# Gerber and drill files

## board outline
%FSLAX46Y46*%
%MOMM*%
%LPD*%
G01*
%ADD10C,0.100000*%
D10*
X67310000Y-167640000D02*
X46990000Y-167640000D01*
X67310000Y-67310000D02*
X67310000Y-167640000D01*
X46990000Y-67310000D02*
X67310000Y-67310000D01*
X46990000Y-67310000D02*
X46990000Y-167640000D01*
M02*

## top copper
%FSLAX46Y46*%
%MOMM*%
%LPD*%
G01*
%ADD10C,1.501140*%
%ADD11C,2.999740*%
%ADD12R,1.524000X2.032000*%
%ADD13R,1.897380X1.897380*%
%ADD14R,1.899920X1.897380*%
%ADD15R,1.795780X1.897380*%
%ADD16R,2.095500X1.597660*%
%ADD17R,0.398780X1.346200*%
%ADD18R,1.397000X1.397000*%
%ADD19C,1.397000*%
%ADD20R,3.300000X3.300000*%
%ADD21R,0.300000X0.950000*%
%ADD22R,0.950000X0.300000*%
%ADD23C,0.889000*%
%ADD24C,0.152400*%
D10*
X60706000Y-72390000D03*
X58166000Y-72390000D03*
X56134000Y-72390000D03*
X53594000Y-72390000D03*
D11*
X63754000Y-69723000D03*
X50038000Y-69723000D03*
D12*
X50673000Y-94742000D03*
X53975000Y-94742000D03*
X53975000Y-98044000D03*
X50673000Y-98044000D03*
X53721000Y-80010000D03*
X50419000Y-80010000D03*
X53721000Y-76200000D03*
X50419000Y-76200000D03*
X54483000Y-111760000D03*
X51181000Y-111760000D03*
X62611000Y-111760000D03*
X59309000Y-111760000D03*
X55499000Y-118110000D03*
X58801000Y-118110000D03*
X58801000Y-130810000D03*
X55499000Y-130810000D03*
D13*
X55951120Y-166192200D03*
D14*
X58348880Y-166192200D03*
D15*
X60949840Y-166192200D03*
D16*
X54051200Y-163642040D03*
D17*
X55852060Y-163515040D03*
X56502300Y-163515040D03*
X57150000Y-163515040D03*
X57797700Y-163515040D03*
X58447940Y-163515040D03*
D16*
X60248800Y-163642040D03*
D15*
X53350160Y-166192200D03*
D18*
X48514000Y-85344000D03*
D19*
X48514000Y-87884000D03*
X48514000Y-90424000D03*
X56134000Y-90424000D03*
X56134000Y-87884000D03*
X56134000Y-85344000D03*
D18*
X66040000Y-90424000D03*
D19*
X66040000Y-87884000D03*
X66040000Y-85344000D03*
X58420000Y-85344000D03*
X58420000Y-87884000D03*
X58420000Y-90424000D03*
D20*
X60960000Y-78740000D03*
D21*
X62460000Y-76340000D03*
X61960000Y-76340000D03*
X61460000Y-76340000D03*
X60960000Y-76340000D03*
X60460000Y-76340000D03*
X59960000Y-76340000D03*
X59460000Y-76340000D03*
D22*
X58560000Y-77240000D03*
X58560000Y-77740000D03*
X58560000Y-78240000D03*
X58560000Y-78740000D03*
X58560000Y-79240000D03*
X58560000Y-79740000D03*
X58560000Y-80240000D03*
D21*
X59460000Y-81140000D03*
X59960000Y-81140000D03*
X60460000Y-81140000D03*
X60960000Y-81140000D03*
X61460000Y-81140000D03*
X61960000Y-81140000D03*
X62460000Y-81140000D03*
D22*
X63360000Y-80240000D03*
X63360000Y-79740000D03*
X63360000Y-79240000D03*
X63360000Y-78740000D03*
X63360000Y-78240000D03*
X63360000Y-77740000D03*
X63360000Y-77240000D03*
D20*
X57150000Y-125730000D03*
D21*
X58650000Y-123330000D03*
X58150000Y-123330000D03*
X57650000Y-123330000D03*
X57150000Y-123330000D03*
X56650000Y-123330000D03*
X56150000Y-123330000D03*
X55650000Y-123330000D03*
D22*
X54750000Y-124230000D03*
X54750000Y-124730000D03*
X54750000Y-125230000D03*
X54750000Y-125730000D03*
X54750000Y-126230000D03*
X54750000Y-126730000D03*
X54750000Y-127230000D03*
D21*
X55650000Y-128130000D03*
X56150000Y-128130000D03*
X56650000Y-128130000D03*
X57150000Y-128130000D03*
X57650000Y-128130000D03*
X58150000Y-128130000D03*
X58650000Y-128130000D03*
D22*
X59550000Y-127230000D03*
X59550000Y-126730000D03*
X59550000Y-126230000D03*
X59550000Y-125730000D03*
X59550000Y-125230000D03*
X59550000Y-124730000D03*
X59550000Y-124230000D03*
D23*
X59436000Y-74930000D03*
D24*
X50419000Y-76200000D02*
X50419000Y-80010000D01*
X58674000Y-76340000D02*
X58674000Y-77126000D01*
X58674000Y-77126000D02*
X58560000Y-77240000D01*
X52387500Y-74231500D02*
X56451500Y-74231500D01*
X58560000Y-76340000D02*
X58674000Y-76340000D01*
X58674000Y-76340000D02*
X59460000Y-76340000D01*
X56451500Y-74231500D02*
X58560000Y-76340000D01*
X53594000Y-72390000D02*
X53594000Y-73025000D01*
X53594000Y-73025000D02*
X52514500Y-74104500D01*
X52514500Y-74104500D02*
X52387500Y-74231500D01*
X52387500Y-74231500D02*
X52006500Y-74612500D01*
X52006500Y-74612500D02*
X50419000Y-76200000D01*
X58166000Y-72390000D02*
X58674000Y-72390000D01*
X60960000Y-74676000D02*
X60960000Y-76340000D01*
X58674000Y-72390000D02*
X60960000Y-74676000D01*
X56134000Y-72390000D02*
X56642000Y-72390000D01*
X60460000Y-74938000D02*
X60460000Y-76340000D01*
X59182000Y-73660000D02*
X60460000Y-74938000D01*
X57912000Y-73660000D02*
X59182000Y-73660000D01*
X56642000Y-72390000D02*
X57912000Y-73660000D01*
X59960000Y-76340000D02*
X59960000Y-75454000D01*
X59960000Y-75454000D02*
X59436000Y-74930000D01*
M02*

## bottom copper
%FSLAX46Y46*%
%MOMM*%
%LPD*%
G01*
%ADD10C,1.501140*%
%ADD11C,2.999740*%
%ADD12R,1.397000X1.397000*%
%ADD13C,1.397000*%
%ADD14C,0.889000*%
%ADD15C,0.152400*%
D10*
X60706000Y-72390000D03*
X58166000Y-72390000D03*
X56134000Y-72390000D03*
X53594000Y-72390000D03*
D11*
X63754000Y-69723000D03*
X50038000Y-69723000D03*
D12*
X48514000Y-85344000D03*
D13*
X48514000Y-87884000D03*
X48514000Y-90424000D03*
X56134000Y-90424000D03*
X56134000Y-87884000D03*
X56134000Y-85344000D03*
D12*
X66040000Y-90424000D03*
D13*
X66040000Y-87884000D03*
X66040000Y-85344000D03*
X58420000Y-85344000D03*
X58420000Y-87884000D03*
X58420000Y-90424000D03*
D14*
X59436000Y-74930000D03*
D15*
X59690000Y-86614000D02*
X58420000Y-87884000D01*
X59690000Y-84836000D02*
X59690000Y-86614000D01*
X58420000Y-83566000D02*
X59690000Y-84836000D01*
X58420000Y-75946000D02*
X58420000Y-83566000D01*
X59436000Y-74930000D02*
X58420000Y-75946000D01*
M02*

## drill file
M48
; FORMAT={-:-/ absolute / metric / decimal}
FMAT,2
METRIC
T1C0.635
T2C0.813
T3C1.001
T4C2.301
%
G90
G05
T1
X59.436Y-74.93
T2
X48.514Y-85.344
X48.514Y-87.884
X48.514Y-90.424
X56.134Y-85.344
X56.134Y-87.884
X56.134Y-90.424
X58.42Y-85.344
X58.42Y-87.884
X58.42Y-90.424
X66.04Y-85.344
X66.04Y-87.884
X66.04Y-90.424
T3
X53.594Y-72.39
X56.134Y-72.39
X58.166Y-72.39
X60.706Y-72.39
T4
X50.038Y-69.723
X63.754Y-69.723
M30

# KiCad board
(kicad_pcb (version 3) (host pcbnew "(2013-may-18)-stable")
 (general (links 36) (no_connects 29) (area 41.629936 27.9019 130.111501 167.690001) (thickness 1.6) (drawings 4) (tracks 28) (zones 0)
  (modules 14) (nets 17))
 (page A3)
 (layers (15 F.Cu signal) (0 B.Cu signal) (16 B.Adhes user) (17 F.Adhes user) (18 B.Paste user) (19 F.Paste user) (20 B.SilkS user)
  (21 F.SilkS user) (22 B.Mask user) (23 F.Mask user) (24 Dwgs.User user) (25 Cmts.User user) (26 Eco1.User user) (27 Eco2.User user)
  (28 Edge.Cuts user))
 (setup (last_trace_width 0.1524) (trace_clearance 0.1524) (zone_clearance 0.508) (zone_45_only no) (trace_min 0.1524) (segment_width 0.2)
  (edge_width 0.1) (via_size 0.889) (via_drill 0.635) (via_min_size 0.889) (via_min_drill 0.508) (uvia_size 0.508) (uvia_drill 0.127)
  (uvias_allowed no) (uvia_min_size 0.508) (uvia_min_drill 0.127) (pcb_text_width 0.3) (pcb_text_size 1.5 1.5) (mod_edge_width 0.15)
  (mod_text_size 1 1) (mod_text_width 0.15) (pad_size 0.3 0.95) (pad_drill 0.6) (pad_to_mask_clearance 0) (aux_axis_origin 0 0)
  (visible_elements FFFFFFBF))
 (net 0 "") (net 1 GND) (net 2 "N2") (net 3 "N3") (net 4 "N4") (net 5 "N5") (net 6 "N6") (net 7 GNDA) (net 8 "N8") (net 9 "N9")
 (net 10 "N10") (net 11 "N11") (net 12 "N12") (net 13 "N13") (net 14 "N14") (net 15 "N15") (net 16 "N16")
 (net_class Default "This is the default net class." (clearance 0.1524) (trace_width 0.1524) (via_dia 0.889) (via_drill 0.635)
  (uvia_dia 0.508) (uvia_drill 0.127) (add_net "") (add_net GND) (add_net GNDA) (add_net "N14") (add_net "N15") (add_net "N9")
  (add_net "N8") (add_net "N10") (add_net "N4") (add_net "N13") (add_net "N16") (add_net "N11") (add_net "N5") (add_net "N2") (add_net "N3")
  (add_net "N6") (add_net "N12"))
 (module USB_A (layer B.Cu) (at 57.15 72.39 90)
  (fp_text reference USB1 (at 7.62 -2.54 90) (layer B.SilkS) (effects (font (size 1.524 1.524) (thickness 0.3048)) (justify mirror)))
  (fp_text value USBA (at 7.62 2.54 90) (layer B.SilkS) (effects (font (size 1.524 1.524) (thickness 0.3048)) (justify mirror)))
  (pad 4 thru_hole circle (at 0 3.556 90) (size 1.50114 1.50114) (drill 1.00076) (layers *.Cu *.Mask B.SilkS) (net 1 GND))
  (pad 3 thru_hole circle (at 0 1.016 90) (size 1.50114 1.50114) (drill 1.00076) (layers *.Cu *.Mask B.SilkS) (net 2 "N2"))
  (pad 2 thru_hole circle (at 0 -1.016 90) (size 1.50114 1.50114) (drill 1.00076) (layers *.Cu *.Mask B.SilkS) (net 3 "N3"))
  (pad 1 thru_hole circle (at 0 -3.556 90) (size 1.50114 1.50114) (drill 1.00076) (layers *.Cu *.Mask B.SilkS) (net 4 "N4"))
  (pad 5 thru_hole circle (at 2.667 6.604 90) (size 2.99974 2.99974) (drill 2.30124) (layers *.Cu *.Mask B.SilkS))
  (pad 6 thru_hole circle (at 2.667 -7.112 90) (size 2.99974 2.99974) (drill 2.30124) (layers *.Cu *.Mask B.SilkS)))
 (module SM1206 (layer F.Cu) (at 52.324 94.742)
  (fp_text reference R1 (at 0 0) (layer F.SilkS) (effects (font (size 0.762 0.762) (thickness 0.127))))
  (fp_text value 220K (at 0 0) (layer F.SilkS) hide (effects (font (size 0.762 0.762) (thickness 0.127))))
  (pad 1 smd rect (at -1.651 0) (size 1.524 2.032) (layers F.Cu F.Paste F.Mask) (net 1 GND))
  (pad 2 smd rect (at 1.651 0) (size 1.524 2.032) (layers F.Cu F.Paste F.Mask) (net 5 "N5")))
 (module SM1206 (layer F.Cu) (at 52.324 98.044 180)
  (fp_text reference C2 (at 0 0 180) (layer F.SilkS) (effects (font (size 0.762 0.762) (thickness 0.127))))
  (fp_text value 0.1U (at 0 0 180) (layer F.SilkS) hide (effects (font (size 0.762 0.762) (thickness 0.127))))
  (pad 1 smd rect (at -1.651 0 180) (size 1.524 2.032) (layers F.Cu F.Paste F.Mask) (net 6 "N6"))
  (pad 2 smd rect (at 1.651 0 180) (size 1.524 2.032) (layers F.Cu F.Paste F.Mask) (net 1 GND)))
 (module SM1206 (layer F.Cu) (at 52.07 80.01 180)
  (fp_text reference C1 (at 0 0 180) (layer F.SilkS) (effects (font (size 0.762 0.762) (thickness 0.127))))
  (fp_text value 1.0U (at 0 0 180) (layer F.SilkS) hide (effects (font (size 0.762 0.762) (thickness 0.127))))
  (pad 1 smd rect (at -1.651 0 180) (size 1.524 2.032) (layers F.Cu F.Paste F.Mask) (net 1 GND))
  (pad 2 smd rect (at 1.651 0 180) (size 1.524 2.032) (layers F.Cu F.Paste F.Mask) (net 4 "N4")))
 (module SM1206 (layer F.Cu) (at 52.07 76.2 180)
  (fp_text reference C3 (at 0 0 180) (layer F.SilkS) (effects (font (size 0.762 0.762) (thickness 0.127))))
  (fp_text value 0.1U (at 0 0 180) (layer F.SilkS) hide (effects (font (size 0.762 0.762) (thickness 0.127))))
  (pad 1 smd rect (at -1.651 0 180) (size 1.524 2.032) (layers F.Cu F.Paste F.Mask) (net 1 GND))
  (pad 2 smd rect (at 1.651 0 180) (size 1.524 2.032) (layers F.Cu F.Paste F.Mask) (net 4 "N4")))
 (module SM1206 (layer F.Cu) (at 52.832 111.76 180)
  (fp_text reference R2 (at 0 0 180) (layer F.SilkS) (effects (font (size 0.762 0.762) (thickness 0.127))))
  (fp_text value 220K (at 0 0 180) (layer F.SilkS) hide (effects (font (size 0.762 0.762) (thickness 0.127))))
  (pad 1 smd rect (at -1.651 0 180) (size 1.524 2.032) (layers F.Cu F.Paste F.Mask) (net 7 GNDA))
  (pad 2 smd rect (at 1.651 0 180) (size 1.524 2.032) (layers F.Cu F.Paste F.Mask) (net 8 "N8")))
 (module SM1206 (layer F.Cu) (at 60.96 111.76 180)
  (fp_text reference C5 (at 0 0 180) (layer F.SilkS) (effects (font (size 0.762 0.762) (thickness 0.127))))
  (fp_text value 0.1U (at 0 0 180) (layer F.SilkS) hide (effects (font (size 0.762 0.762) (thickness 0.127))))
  (pad 1 smd rect (at -1.651 0 180) (size 1.524 2.032) (layers F.Cu F.Paste F.Mask) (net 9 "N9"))
  (pad 2 smd rect (at 1.651 0 180) (size 1.524 2.032) (layers F.Cu F.Paste F.Mask) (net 7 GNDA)))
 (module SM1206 (layer F.Cu) (at 57.15 118.11)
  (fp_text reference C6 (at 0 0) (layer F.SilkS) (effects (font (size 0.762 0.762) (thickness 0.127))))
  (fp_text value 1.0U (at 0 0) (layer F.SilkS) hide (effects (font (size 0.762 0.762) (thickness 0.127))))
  (pad 1 smd rect (at -1.651 0) (size 1.524 2.032) (layers F.Cu F.Paste F.Mask) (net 7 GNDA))
  (pad 2 smd rect (at 1.651 0) (size 1.524 2.032) (layers F.Cu F.Paste F.Mask) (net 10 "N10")))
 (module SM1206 (layer F.Cu) (at 57.15 130.81 180)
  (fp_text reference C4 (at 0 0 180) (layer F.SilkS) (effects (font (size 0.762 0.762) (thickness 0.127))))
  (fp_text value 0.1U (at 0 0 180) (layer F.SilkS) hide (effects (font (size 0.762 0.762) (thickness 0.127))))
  (pad 1 smd rect (at -1.651 0 180) (size 1.524 2.032) (layers F.Cu F.Paste F.Mask) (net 7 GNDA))
  (pad 2 smd rect (at 1.651 0 180) (size 1.524 2.032) (layers F.Cu F.Paste F.Mask) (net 10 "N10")))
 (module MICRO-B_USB (layer F.Cu) (at 57.15 167.64)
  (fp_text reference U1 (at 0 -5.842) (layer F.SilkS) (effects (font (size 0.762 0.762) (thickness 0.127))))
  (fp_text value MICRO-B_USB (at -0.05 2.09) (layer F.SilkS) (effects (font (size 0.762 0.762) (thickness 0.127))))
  (pad "" smd rect (at -1.19888 -1.4478) (size 1.89738 1.89738) (layers F.Cu F.Paste F.Mask))
  (pad "" smd rect (at 1.19888 -1.4478) (size 1.89992 1.89738) (layers F.Cu F.Paste F.Mask))
  (pad "" smd rect (at 3.79984 -1.4478) (size 1.79578 1.89738) (layers F.Cu F.Paste F.Mask))
  (pad "" smd rect (at -3.0988 -3.99796) (size 2.0955 1.59766) (layers F.Cu F.Paste F.Mask))
  (pad 1 smd rect (at -1.29794 -4.12496) (size 0.39878 1.3462) (layers F.Cu F.Paste F.Mask) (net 10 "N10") (clearance 0.2032))
  (pad 2 smd rect (at -0.6477 -4.12496) (size 0.39878 1.3462) (layers F.Cu F.Paste F.Mask) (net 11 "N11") (clearance 0.2032))
  (pad 3 smd rect (at 0 -4.12496) (size 0.39878 1.3462) (layers F.Cu F.Paste F.Mask) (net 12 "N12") (clearance 0.2032))
  (pad 4 smd rect (at 0.6477 -4.12496) (size 0.39878 1.3462) (layers F.Cu F.Paste F.Mask) (clearance 0.2032))
  (pad 5 smd rect (at 1.29794 -4.12496) (size 0.39878 1.3462) (layers F.Cu F.Paste F.Mask) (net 7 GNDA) (clearance 0.2032))
  (pad "" smd rect (at 3.0988 -3.99796) (size 2.0955 1.59766) (layers F.Cu F.Paste F.Mask))
  (pad "" smd rect (at -3.79984 -1.4478) (size 1.79578 1.89738) (layers F.Cu F.Paste F.Mask)))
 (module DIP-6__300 (layer F.Cu) (at 52.324 87.884 270)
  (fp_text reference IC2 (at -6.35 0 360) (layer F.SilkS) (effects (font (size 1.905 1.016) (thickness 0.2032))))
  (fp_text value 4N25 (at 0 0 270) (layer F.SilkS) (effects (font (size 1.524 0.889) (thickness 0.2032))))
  (pad 1 thru_hole rect (at -2.54 3.81 270) (size 1.397 1.397) (drill 0.8128) (layers *.Cu *.Mask F.SilkS) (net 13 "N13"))
  (pad 2 thru_hole circle (at 0 3.81 270) (size 1.397 1.397) (drill 0.8128) (layers *.Cu *.Mask F.SilkS) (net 1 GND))
  (pad 3 thru_hole circle (at 2.54 3.81 270) (size 1.397 1.397) (drill 0.8128) (layers *.Cu *.Mask F.SilkS))
  (pad 4 thru_hole circle (at 2.54 -3.81 270) (size 1.397 1.397) (drill 0.8128) (layers *.Cu *.Mask F.SilkS) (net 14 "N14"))
  (pad 5 thru_hole circle (at 0 -3.81 270) (size 1.397 1.397) (drill 0.8128) (layers *.Cu *.Mask F.SilkS) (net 9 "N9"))
  (pad 6 thru_hole circle (at -2.54 -3.81 270) (size 1.397 1.397) (drill 0.8128) (layers *.Cu *.Mask F.SilkS) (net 8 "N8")))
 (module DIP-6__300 (layer F.Cu) (at 62.23 87.884 90)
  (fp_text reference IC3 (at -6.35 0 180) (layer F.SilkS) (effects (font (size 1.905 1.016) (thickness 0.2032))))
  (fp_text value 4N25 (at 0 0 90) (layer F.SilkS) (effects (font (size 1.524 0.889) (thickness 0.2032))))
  (pad 1 thru_hole rect (at -2.54 3.81 90) (size 1.397 1.397) (drill 0.8128) (layers *.Cu *.Mask F.SilkS) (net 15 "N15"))
  (pad 2 thru_hole circle (at 0 3.81 90) (size 1.397 1.397) (drill 0.8128) (layers *.Cu *.Mask F.SilkS) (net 7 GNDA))
  (pad 3 thru_hole circle (at 2.54 3.81 90) (size 1.397 1.397) (drill 0.8128) (layers *.Cu *.Mask F.SilkS))
  (pad 4 thru_hole circle (at 2.54 -3.81 90) (size 1.397 1.397) (drill 0.8128) (layers *.Cu *.Mask F.SilkS) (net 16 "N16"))
  (pad 5 thru_hole circle (at 0 -3.81 90) (size 1.397 1.397) (drill 0.8128) (layers *.Cu *.Mask F.SilkS) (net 6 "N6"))
  (pad 6 thru_hole circle (at -2.54 -3.81 90) (size 1.397 1.397) (drill 0.8128) (layers *.Cu *.Mask F.SilkS) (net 5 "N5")))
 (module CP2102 (layer F.Cu) (at 60.96 78.74 270)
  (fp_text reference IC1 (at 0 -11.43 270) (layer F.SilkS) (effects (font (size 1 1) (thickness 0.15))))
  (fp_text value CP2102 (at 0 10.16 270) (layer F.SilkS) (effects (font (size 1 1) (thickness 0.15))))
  (pad 3 smd rect (at 0 0 270) (size 3.3 3.3) (layers F.Cu F.Paste F.Mask) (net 1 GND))
  (pad 1 smd rect (at -2.4 -1.5 270) (size 0.95 0.3) (layers F.Cu F.Paste F.Mask))
  (pad 2 smd rect (at -2.4 -1 270) (size 0.95 0.3) (layers F.Cu F.Paste F.Mask))
  (pad 3 smd rect (at -2.4 -0.5 270) (size 0.95 0.3) (layers F.Cu F.Paste F.Mask) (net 1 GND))
  (pad 4 smd rect (at -2.4 0 270) (size 0.95 0.3) (layers F.Cu F.Paste F.Mask) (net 2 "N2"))
  (pad 5 smd rect (at -2.4 0.5 270) (size 0.95 0.3) (layers F.Cu F.Paste F.Mask) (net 3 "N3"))
  (pad 6 smd rect (at -2.4 1 270) (size 0.95 0.3) (layers F.Cu F.Paste F.Mask) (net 6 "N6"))
  (pad 7 smd rect (at -2.4 1.5 270) (size 0.95 0.3) (layers F.Cu F.Paste F.Mask) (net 4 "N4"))
  (pad 8 smd rect (at -1.5 2.4 270) (size 0.3 0.95) (layers F.Cu F.Paste F.Mask) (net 4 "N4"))
  (pad 9 smd rect (at -1 2.4 270) (size 0.3 0.95) (layers F.Cu F.Paste F.Mask))
  (pad 10 smd rect (at -0.5 2.4 270) (size 0.3 0.95) (layers F.Cu F.Paste F.Mask))
  (pad 11 smd rect (at 0 2.4 270) (size 0.3 0.95) (layers F.Cu F.Paste F.Mask))
  (pad 12 smd rect (at 0.5 2.4 270) (size 0.3 0.95) (layers F.Cu F.Paste F.Mask))
  (pad 13 smd rect (at 1 2.4 270) (size 0.3 0.95) (layers F.Cu F.Paste F.Mask))
  (pad 14 smd rect (at 1.5 2.4 270) (size 0.3 0.95) (layers F.Cu F.Paste F.Mask))
  (pad 15 smd rect (at 2.4 1.5 270) (size 0.95 0.3) (layers F.Cu F.Paste F.Mask))
  (pad 16 smd rect (at 2.4 1 270) (size 0.95 0.3) (layers F.Cu F.Paste F.Mask))
  (pad 17 smd rect (at 2.4 0.5 270) (size 0.95 0.3) (layers F.Cu F.Paste F.Mask))
  (pad 18 smd rect (at 2.4 0 270) (size 0.95 0.3) (layers F.Cu F.Paste F.Mask))
  (pad 19 smd rect (at 2.4 -0.5 270) (size 0.95 0.3) (layers F.Cu F.Paste F.Mask))
  (pad 20 smd rect (at 2.4 -1 270) (size 0.95 0.3) (layers F.Cu F.Paste F.Mask))
  (pad 21 smd rect (at 2.4 -1.5 270) (size 0.95 0.3) (layers F.Cu F.Paste F.Mask))
  (pad 22 smd rect (at 1.5 -2.4 270) (size 0.3 0.95) (layers F.Cu F.Paste F.Mask))
  (pad 23 smd rect (at 1 -2.4 270) (size 0.3 0.95) (layers F.Cu F.Paste F.Mask))
  (pad 24 smd rect (at 0.5 -2.4 270) (size 0.3 0.95) (layers F.Cu F.Paste F.Mask))
  (pad 25 smd rect (at 0 -2.4 270) (size 0.3 0.95) (layers F.Cu F.Paste F.Mask) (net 16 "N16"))
  (pad 26 smd rect (at -0.5 -2.4 270) (size 0.3 0.95) (layers F.Cu F.Paste F.Mask) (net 13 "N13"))
  (pad 27 smd rect (at -1 -2.4 270) (size 0.3 0.95) (layers F.Cu F.Paste F.Mask))
  (pad 28 smd rect (at -1.5 -2.4 270) (size 0.3 0.95) (layers F.Cu F.Paste F.Mask)))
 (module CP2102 (layer F.Cu) (at 57.15 125.73 270)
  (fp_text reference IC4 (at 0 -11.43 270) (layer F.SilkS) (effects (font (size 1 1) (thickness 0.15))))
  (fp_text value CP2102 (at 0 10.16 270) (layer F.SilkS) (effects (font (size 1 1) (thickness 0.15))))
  (pad 3 smd rect (at 0 0 270) (size 3.3 3.3) (layers F.Cu F.Paste F.Mask) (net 7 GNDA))
  (pad 1 smd rect (at -2.4 -1.5 270) (size 0.95 0.3) (layers F.Cu F.Paste F.Mask))
  (pad 2 smd rect (at -2.4 -1 270) (size 0.95 0.3) (layers F.Cu F.Paste F.Mask))
  (pad 3 smd rect (at -2.4 -0.5 270) (size 0.95 0.3) (layers F.Cu F.Paste F.Mask) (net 7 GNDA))
  (pad 4 smd rect (at -2.4 0 270) (size 0.95 0.3) (layers F.Cu F.Paste F.Mask) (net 12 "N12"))
  (pad 5 smd rect (at -2.4 0.5 270) (size 0.95 0.3) (layers F.Cu F.Paste F.Mask) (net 11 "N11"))
  (pad 6 smd rect (at -2.4 1 270) (size 0.95 0.3) (layers F.Cu F.Paste F.Mask) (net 9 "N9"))
  (pad 7 smd rect (at -2.4 1.5 270) (size 0.95 0.3) (layers F.Cu F.Paste F.Mask) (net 10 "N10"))
  (pad 8 smd rect (at -1.5 2.4 270) (size 0.3 0.95) (layers F.Cu F.Paste F.Mask) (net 10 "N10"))
  (pad 9 smd rect (at -1 2.4 270) (size 0.3 0.95) (layers F.Cu F.Paste F.Mask))
  (pad 10 smd rect (at -0.5 2.4 270) (size 0.3 0.95) (layers F.Cu F.Paste F.Mask))
  (pad 11 smd rect (at 0 2.4 270) (size 0.3 0.95) (layers F.Cu F.Paste F.Mask))
  (pad 12 smd rect (at 0.5 2.4 270) (size 0.3 0.95) (layers F.Cu F.Paste F.Mask))
  (pad 13 smd rect (at 1 2.4 270) (size 0.3 0.95) (layers F.Cu F.Paste F.Mask))
  (pad 14 smd rect (at 1.5 2.4 270) (size 0.3 0.95) (layers F.Cu F.Paste F.Mask))
  (pad 15 smd rect (at 2.4 1.5 270) (size 0.95 0.3) (layers F.Cu F.Paste F.Mask))
  (pad 16 smd rect (at 2.4 1 270) (size 0.95 0.3) (layers F.Cu F.Paste F.Mask))
  (pad 17 smd rect (at 2.4 0.5 270) (size 0.95 0.3) (layers F.Cu F.Paste F.Mask))
  (pad 18 smd rect (at 2.4 0 270) (size 0.95 0.3) (layers F.Cu F.Paste F.Mask))
  (pad 19 smd rect (at 2.4 -0.5 270) (size 0.95 0.3) (layers F.Cu F.Paste F.Mask))
  (pad 20 smd rect (at 2.4 -1 270) (size 0.95 0.3) (layers F.Cu F.Paste F.Mask))
  (pad 21 smd rect (at 2.4 -1.5 270) (size 0.95 0.3) (layers F.Cu F.Paste F.Mask))
  (pad 22 smd rect (at 1.5 -2.4 270) (size 0.3 0.95) (layers F.Cu F.Paste F.Mask))
  (pad 23 smd rect (at 1 -2.4 270) (size 0.3 0.95) (layers F.Cu F.Paste F.Mask))
  (pad 24 smd rect (at 0.5 -2.4 270) (size 0.3 0.95) (layers F.Cu F.Paste F.Mask))
  (pad 25 smd rect (at 0 -2.4 270) (size 0.3 0.95) (layers F.Cu F.Paste F.Mask) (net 14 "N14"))
  (pad 26 smd rect (at -0.5 -2.4 270) (size 0.3 0.95) (layers F.Cu F.Paste F.Mask) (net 15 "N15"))
  (pad 27 smd rect (at -1 -2.4 270) (size 0.3 0.95) (layers F.Cu F.Paste F.Mask))
  (pad 28 smd rect (at -1.5 -2.4 270) (size 0.3 0.95) (layers F.Cu F.Paste F.Mask)))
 (gr_line (start 67.31 167.64) (end 46.99 167.64) (angle 90) (layer Edge.Cuts) (width 0.1))
 (gr_line (start 67.31 67.31) (end 67.31 167.64) (angle 90) (layer Edge.Cuts) (width 0.1))
 (gr_line (start 46.99 67.31) (end 67.31 67.31) (angle 90) (layer Edge.Cuts) (width 0.1))
 (gr_line (start 46.99 67.31) (end 46.99 167.64) (angle 90) (layer Edge.Cuts) (width 0.1))
 (segment (start 50.419 76.2) (end 50.419 80.01) (width 0.1524) (layer F.Cu) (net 4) (status C00000))
 (segment (start 58.674 76.34) (end 58.674 77.126) (width 0.1524) (layer F.Cu) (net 4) (status 800000))
 (segment (start 58.674 77.126) (end 58.56 77.24) (width 0.1524) (layer F.Cu) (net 4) (status C00000))
 (segment (start 52.3875 74.2315) (end 56.4515 74.2315) (width 0.1524) (layer F.Cu) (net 4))
 (segment (start 58.56 76.34) (end 58.674 76.34) (width 0.1524) (layer F.Cu) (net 4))
 (segment (start 58.674 76.34) (end 59.46 76.34) (width 0.1524) (layer F.Cu) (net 4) (status 800000))
 (segment (start 56.4515 74.2315) (end 58.56 76.34) (width 0.1524) (layer F.Cu) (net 4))
 (segment (start 53.594 72.39) (end 53.594 73.025) (width 0.1524) (layer F.Cu) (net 4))
 (segment (start 53.594 73.025) (end 52.5145 74.1045) (width 0.1524) (layer F.Cu) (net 4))
 (segment (start 52.5145 74.1045) (end 52.3875 74.2315) (width 0.1524) (layer F.Cu) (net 4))
 (segment (start 52.3875 74.2315) (end 52.0065 74.6125) (width 0.1524) (layer F.Cu) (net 4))
 (segment (start 52.0065 74.6125) (end 50.419 76.2) (width 0.1524) (layer F.Cu) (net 4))
 (segment (start 58.166 72.39) (end 58.674 72.39) (width 0.1524) (layer F.Cu) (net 2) (status C00000))
 (segment (start 60.96 74.676) (end 60.96 76.34) (width 0.1524) (layer F.Cu) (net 2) (status 800000))
 (segment (start 58.674 72.39) (end 60.96 74.676) (width 0.1524) (layer F.Cu) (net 2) (status 400000))
 (segment (start 56.134 72.39) (end 56.642 72.39) (width 0.1524) (layer F.Cu) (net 3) (status C00000))
 (segment (start 60.46 74.938) (end 60.46 76.34) (width 0.1524) (layer F.Cu) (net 3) (status 800000))
 (segment (start 59.182 73.66) (end 60.46 74.938) (width 0.1524) (layer F.Cu) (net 3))
 (segment (start 57.912 73.66) (end 59.182 73.66) (width 0.1524) (layer F.Cu) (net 3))
 (segment (start 56.642 72.39) (end 57.912 73.66) (width 0.1524) (layer F.Cu) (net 3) (status 400000))
 (segment (start 59.96 76.34) (end 59.96 75.454) (width 0.1524) (layer F.Cu) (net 6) (status 400000))
 (segment (start 59.69 86.614) (end 58.42 87.884) (width 0.1524) (layer B.Cu) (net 6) (status 800000))
 (segment (start 59.69 84.836) (end 59.69 86.614) (width 0.1524) (layer B.Cu) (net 6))
 (segment (start 58.42 83.566) (end 59.69 84.836) (width 0.1524) (layer B.Cu) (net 6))
 (segment (start 58.42 75.946) (end 58.42 83.566) (width 0.1524) (layer B.Cu) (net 6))
 (segment (start 59.436 74.93) (end 58.42 75.946) (width 0.1524) (layer B.Cu) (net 6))
 (via (at 59.436 74.93) (size 0.889) (layers F.Cu B.Cu) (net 6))
 (segment (start 59.96 75.454) (end 59.436 74.93) (width 0.1524) (layer F.Cu) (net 6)))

